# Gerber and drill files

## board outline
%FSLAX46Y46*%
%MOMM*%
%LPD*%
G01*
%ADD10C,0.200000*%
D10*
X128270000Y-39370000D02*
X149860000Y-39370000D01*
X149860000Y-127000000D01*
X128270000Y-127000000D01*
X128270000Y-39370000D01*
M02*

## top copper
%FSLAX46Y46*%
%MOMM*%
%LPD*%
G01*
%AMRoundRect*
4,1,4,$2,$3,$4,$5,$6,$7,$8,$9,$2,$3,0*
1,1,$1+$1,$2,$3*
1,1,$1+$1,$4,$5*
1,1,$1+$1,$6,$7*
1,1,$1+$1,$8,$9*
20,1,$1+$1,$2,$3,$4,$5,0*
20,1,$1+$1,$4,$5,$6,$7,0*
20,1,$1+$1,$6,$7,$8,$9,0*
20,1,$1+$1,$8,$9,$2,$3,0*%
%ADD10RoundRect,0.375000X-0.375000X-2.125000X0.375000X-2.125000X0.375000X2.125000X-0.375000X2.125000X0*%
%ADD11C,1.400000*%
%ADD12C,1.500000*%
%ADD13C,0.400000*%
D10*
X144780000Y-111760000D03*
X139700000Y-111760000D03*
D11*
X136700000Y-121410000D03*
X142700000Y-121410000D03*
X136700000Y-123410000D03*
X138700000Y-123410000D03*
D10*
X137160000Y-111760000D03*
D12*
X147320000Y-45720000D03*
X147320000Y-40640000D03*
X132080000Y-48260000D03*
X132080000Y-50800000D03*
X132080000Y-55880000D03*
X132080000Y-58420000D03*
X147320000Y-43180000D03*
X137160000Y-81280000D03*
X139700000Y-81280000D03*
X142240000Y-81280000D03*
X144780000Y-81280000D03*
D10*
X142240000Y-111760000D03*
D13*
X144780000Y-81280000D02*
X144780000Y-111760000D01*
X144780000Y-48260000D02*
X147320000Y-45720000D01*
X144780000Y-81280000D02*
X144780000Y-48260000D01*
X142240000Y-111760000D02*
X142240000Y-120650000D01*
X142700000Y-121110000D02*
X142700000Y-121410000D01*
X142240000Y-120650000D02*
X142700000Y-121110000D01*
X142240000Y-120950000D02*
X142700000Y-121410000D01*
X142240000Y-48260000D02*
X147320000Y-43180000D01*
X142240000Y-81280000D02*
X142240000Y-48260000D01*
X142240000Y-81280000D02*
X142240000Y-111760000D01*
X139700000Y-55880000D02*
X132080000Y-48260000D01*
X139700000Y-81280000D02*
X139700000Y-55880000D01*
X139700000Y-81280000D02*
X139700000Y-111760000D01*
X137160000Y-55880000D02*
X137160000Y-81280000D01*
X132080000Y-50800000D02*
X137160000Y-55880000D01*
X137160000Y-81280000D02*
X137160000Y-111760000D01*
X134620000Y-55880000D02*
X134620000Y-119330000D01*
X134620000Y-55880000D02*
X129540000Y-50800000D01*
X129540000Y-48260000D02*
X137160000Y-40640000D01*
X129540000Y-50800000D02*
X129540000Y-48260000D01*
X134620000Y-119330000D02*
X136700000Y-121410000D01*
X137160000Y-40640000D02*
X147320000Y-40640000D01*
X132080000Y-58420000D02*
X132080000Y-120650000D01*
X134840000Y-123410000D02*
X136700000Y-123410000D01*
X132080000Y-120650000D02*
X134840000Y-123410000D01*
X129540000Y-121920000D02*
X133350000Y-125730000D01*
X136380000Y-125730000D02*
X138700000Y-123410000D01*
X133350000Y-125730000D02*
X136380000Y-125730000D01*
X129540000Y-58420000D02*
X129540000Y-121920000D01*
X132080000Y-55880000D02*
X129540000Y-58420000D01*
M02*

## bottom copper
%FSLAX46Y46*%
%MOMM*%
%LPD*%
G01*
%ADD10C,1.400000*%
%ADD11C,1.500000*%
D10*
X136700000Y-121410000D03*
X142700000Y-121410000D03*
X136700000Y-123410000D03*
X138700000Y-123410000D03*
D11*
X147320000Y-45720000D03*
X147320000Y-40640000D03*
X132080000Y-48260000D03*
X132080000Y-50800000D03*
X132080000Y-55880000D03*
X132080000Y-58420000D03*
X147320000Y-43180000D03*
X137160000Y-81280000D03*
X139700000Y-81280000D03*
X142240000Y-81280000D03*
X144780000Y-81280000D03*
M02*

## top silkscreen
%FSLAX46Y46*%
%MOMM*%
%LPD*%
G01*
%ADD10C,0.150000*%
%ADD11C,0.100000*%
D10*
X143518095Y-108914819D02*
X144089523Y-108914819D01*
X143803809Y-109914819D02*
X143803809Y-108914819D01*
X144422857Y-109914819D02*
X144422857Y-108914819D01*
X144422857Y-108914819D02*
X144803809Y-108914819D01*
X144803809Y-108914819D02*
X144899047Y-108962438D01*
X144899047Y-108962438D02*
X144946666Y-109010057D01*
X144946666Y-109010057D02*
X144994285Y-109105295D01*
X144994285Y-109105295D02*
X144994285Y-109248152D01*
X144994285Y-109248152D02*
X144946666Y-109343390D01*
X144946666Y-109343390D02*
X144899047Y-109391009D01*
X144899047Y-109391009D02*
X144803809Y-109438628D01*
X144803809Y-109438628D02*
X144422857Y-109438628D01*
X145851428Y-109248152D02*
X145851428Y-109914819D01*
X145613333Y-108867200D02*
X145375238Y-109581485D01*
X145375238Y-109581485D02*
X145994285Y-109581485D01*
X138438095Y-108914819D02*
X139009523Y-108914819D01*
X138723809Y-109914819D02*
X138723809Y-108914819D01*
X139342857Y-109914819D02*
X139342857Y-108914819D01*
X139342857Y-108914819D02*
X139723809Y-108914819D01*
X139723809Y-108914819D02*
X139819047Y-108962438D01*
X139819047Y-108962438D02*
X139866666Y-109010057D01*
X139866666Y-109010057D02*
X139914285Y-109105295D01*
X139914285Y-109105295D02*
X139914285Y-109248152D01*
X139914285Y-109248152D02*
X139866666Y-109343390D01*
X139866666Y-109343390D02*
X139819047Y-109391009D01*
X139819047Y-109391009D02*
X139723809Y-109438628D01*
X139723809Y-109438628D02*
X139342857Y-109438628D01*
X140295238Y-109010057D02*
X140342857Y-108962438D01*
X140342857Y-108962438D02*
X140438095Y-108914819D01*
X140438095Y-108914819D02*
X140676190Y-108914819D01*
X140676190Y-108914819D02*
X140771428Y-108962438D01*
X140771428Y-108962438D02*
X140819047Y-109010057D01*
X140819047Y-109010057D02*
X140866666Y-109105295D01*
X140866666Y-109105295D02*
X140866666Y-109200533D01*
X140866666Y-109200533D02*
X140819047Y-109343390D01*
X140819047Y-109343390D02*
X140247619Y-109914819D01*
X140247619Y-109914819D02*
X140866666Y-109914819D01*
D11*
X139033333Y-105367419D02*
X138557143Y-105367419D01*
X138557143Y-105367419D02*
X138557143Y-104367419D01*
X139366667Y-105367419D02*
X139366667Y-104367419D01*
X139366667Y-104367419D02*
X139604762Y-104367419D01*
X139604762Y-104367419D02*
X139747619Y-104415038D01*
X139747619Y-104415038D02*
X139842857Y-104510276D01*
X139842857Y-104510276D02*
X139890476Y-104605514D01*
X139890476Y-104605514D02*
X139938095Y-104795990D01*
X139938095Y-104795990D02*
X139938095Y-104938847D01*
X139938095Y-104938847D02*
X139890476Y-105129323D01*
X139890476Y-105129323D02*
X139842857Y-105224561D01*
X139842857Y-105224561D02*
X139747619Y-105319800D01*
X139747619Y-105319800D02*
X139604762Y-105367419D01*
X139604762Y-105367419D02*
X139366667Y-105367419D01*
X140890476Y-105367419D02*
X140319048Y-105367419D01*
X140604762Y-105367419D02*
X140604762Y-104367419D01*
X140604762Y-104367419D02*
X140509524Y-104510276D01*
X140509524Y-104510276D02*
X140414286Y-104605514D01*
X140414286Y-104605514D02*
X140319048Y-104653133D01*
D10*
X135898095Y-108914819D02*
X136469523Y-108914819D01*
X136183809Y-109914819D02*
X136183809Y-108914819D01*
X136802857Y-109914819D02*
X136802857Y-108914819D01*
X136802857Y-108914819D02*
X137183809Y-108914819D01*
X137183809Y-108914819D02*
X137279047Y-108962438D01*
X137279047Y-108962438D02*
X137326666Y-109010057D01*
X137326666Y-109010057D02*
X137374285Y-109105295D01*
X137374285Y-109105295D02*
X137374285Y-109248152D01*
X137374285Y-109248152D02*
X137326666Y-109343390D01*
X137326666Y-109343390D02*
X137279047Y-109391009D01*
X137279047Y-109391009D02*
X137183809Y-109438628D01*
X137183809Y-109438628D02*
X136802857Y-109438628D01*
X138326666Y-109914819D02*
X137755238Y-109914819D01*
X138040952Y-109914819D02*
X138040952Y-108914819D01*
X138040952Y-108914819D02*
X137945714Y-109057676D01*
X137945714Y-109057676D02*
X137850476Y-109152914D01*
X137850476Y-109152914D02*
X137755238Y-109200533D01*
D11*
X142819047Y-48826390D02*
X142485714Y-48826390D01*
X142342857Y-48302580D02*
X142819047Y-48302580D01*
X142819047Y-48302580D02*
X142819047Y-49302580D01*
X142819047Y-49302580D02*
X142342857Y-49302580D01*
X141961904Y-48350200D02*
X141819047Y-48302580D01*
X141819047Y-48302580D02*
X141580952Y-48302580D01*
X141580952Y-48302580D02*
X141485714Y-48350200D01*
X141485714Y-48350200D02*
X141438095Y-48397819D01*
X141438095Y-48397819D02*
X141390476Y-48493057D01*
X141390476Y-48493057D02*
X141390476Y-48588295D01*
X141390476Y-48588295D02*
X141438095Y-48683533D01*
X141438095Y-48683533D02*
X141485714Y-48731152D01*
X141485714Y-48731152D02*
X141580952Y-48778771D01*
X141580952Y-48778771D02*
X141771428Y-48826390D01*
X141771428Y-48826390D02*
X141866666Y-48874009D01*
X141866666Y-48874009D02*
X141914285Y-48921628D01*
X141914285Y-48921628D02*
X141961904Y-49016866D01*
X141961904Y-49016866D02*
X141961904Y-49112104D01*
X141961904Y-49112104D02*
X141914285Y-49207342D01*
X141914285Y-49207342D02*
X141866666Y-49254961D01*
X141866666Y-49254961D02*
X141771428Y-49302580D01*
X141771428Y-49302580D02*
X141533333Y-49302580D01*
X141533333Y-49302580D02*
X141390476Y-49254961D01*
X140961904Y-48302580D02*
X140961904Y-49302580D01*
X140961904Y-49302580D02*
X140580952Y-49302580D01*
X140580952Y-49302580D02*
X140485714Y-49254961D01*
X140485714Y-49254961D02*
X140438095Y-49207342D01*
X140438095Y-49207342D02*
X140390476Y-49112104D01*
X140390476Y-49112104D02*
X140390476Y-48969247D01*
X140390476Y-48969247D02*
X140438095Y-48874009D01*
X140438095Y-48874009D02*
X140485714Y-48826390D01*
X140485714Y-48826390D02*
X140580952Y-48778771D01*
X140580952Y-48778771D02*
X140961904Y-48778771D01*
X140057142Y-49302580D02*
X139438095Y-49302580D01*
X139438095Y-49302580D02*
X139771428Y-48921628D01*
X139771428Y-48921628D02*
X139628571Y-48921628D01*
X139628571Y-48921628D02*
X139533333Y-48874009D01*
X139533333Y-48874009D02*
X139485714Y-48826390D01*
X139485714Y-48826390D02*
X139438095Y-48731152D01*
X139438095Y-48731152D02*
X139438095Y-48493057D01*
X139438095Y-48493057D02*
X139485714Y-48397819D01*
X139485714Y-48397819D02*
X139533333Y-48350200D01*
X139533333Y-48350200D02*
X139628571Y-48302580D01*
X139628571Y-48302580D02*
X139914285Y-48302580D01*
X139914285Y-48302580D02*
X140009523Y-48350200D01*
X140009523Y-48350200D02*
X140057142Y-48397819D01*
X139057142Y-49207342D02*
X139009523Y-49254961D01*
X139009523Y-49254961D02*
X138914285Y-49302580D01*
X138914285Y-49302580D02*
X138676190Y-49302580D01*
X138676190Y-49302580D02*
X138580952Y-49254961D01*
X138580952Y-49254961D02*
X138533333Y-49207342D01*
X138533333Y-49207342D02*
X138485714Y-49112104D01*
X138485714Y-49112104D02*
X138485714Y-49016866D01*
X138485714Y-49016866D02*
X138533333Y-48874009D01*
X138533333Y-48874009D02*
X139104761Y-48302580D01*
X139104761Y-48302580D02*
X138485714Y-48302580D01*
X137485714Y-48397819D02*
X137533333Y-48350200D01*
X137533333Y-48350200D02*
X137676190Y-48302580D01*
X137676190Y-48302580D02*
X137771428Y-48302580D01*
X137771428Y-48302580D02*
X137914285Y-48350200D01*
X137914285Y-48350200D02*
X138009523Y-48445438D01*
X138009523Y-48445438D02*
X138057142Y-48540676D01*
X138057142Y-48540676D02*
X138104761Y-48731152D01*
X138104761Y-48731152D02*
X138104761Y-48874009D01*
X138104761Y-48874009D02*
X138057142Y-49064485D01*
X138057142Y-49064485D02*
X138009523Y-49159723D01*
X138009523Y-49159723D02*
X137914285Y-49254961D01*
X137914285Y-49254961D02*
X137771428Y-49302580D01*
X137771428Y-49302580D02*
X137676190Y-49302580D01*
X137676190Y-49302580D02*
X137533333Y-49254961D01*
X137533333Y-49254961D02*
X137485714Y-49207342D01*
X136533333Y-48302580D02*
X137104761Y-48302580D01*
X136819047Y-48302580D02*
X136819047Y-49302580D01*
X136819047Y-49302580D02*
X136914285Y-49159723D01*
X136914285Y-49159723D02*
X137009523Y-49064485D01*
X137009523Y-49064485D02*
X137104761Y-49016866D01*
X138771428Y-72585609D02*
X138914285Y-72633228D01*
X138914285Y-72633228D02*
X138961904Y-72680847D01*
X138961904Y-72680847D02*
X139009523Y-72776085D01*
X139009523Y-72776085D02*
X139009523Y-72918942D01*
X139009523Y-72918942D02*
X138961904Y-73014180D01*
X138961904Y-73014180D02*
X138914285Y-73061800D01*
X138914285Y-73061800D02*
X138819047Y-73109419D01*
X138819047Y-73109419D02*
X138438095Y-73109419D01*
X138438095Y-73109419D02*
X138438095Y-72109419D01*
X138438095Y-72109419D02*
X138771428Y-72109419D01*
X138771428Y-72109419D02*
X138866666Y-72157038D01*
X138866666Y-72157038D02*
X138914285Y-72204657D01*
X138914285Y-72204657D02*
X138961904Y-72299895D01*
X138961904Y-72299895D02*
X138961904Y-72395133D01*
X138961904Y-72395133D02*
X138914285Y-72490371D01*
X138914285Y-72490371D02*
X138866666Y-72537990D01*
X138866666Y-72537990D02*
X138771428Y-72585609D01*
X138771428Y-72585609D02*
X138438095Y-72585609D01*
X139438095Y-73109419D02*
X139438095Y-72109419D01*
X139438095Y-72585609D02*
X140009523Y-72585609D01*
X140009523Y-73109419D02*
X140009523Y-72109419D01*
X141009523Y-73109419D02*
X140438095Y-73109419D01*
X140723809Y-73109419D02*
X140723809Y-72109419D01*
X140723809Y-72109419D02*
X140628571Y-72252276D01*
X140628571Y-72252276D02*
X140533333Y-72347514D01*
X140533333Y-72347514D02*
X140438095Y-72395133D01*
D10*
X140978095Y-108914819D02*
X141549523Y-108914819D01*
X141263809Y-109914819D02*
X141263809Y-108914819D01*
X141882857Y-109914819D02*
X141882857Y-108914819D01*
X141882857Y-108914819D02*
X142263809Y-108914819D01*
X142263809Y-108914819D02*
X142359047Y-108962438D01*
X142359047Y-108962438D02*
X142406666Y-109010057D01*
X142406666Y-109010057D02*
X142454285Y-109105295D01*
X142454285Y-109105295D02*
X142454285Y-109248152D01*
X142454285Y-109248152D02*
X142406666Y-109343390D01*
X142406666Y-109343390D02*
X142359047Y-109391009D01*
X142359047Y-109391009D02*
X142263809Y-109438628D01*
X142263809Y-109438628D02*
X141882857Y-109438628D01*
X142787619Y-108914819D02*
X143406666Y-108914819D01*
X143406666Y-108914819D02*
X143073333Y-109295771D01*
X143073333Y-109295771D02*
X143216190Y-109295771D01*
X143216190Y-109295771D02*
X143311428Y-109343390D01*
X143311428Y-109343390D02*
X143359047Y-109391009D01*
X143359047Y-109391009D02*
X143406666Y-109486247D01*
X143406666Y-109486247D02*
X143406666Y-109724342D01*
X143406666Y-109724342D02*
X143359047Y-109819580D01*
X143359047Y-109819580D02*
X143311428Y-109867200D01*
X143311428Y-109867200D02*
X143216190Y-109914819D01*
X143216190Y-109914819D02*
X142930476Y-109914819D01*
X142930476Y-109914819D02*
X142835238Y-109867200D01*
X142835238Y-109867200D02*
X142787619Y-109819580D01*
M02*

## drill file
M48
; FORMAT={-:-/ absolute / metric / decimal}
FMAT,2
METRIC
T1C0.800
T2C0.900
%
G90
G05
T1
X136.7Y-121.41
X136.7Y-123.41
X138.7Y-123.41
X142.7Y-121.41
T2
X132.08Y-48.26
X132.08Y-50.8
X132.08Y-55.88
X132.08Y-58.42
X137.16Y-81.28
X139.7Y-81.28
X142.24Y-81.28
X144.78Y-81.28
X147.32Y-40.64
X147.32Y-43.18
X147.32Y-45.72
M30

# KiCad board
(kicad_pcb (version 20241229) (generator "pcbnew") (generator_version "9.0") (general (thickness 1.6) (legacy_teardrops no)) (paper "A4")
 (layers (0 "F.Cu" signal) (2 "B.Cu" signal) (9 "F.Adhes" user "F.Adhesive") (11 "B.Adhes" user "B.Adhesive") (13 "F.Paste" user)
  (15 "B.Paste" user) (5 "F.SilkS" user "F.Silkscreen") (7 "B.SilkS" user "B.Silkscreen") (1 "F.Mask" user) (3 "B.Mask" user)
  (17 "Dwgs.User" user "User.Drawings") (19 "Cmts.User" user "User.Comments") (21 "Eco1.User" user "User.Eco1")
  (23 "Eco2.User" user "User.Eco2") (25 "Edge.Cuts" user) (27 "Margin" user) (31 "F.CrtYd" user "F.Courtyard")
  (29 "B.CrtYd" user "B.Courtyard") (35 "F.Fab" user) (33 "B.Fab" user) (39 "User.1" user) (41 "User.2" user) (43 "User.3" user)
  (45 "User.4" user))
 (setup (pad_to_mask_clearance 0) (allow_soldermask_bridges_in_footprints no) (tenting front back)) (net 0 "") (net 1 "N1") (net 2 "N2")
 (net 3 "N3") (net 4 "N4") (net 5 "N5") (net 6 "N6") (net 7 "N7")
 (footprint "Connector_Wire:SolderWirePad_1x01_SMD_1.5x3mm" (layer "F.Cu") (at 144.78 111.76)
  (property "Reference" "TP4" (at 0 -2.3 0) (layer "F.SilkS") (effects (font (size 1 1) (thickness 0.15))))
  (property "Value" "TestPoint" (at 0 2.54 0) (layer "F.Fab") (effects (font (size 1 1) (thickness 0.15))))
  (pad "1" smd roundrect (at 0 0) (size 1.5 5) (layers "F.Cu" "F.Mask") (roundrect_rratio 0.25) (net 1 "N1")))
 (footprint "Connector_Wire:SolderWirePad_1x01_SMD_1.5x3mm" (layer "F.Cu") (at 139.7 111.76)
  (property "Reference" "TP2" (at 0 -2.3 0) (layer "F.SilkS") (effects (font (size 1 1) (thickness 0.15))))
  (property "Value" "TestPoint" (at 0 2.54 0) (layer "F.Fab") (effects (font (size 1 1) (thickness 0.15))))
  (pad "1" smd roundrect (at 0 0) (size 1.5 5) (layers "F.Cu" "F.Mask") (roundrect_rratio 0.25) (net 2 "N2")))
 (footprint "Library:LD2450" (layer "F.Cu") (at 139.7 105.41)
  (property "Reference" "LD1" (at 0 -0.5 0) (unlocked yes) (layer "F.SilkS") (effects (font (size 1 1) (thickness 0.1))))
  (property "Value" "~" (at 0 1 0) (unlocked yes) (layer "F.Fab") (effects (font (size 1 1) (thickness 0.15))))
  (pad "1" thru_hole circle (at -3 16 90) (size 1.4 1.4) (drill 0.8) (layers "*.Cu" "*.Mask") (remove_unused_layers yes)
   (keep_end_layers yes) (zone_layer_connections) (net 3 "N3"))
  (pad "2" thru_hole circle (at 3 16 90) (size 1.4 1.4) (drill 0.8) (layers "*.Cu" "*.Mask") (remove_unused_layers yes)
   (keep_end_layers yes) (zone_layer_connections) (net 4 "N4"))
  (pad "3" thru_hole circle (at -3 18 90) (size 1.4 1.4) (drill 0.8) (layers "*.Cu" "*.Mask") (remove_unused_layers yes)
   (keep_end_layers yes) (zone_layer_connections) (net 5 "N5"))
  (pad "4" thru_hole circle (at -1 18 90) (size 1.4 1.4) (drill 0.8) (layers "*.Cu" "*.Mask") (remove_unused_layers yes)
   (keep_end_layers yes) (zone_layer_connections) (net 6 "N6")))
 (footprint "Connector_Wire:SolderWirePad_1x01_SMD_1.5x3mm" (layer "F.Cu") (at 137.16 111.76)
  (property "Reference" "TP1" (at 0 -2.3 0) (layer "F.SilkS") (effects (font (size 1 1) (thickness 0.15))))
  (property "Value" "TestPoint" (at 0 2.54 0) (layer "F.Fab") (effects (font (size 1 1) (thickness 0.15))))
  (pad "1" smd roundrect (at 0 0) (size 1.5 5) (layers "F.Cu" "F.Mask") (roundrect_rratio 0.25) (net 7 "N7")))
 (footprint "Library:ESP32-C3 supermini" (layer "F.Cu") (at 139.7 50.8 180)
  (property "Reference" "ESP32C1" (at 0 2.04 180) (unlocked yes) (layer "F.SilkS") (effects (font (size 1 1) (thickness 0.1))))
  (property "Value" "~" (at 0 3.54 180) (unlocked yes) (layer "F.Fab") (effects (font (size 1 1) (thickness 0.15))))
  (pad "3.3V" thru_hole circle (at -7.62 5.08 180) (size 1.5 1.5) (drill 0.9) (layers "*.Cu" "*.Mask") (remove_unused_layers yes)
   (keep_end_layers yes) (zone_layer_connections) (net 1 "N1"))
  (pad "5V" thru_hole circle (at -7.62 10.16 180) (size 1.5 1.5) (drill 0.9) (layers "*.Cu" "*.Mask") (remove_unused_layers yes)
   (keep_end_layers yes) (zone_layer_connections) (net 3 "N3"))
  (pad "8" thru_hole circle (at 7.62 2.54 180) (size 1.5 1.5) (drill 0.9) (layers "*.Cu" "*.Mask") (remove_unused_layers yes)
   (keep_end_layers yes) (zone_layer_connections) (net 2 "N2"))
  (pad "9" thru_hole circle (at 7.62 0 180) (size 1.5 1.5) (drill 0.9) (layers "*.Cu" "*.Mask") (remove_unused_layers yes)
   (keep_end_layers yes) (zone_layer_connections) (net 7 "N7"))
  (pad "20" thru_hole circle (at 7.62 -5.08 180) (size 1.5 1.5) (drill 0.9) (layers "*.Cu" "*.Mask") (remove_unused_layers yes)
   (keep_end_layers yes) (zone_layer_connections) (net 6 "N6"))
  (pad "21" thru_hole circle (at 7.62 -7.62 180) (size 1.5 1.5) (drill 0.9) (layers "*.Cu" "*.Mask") (remove_unused_layers yes)
   (keep_end_layers yes) (zone_layer_connections) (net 5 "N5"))
  (pad "GND" thru_hole circle (at -7.62 7.62 180) (size 1.5 1.5) (drill 0.9) (layers "*.Cu" "*.Mask") (remove_unused_layers yes)
   (keep_end_layers yes) (zone_layer_connections) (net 4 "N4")))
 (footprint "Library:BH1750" (layer "F.Cu") (at 139.7 73.152)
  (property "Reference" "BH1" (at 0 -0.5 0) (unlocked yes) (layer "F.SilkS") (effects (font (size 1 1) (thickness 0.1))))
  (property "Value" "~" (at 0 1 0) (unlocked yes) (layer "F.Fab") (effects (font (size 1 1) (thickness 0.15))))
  (pad "1" thru_hole circle (at -2.54 8.128 90) (size 1.5 1.5) (drill 0.9) (layers "*.Cu" "*.Mask") (remove_unused_layers yes)
   (keep_end_layers yes) (zone_layer_connections) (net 7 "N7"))
  (pad "2" thru_hole circle (at 0 8.128 90) (size 1.5 1.5) (drill 0.9) (layers "*.Cu" "*.Mask") (remove_unused_layers yes)
   (keep_end_layers yes) (zone_layer_connections) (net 2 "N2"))
  (pad "3" thru_hole circle (at 2.54 8.128 90) (size 1.5 1.5) (drill 0.9) (layers "*.Cu" "*.Mask") (remove_unused_layers yes)
   (keep_end_layers yes) (zone_layer_connections) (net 4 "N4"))
  (pad "4" thru_hole circle (at 5.08 8.128 90) (size 1.5 1.5) (drill 0.9) (layers "*.Cu" "*.Mask") (remove_unused_layers yes)
   (keep_end_layers yes) (zone_layer_connections) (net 1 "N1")))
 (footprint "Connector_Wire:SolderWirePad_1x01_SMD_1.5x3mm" (layer "F.Cu") (at 142.24 111.76)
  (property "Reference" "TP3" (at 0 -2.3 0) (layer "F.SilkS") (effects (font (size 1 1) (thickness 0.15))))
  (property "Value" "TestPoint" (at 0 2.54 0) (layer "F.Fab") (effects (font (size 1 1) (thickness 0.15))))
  (pad "1" smd roundrect (at 0 0) (size 1.5 5) (layers "F.Cu" "F.Mask") (roundrect_rratio 0.25) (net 4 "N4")))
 (gr_rect (start 128.27 39.37) (end 149.86 127) (stroke (width 0.2) (type solid)) (fill no) (layer "Edge.Cuts"))
 (segment (start 144.78 81.28) (end 144.78 111.76) (width 0.4) (layer "F.Cu") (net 1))
 (segment (start 144.78 48.26) (end 147.32 45.72) (width 0.4) (layer "F.Cu") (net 1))
 (segment (start 144.78 81.28) (end 144.78 48.26) (width 0.4) (layer "F.Cu") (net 1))
 (segment (start 142.24 111.76) (end 142.24 120.65) (width 0.4) (layer "F.Cu") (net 4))
 (segment (start 142.7 121.11) (end 142.7 121.41) (width 0.4) (layer "F.Cu") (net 4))
 (segment (start 142.24 120.65) (end 142.7 121.11) (width 0.4) (layer "F.Cu") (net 4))
 (segment (start 142.24 120.95) (end 142.7 121.41) (width 0.4) (layer "F.Cu") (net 4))
 (segment (start 142.24 48.26) (end 147.32 43.18) (width 0.4) (layer "F.Cu") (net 4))
 (segment (start 142.24 81.28) (end 142.24 48.26) (width 0.4) (layer "F.Cu") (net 4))
 (segment (start 142.24 81.28) (end 142.24 111.76) (width 0.4) (layer "F.Cu") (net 4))
 (segment (start 139.7 55.88) (end 132.08 48.26) (width 0.4) (layer "F.Cu") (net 2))
 (segment (start 139.7 81.28) (end 139.7 55.88) (width 0.4) (layer "F.Cu") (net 2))
 (segment (start 139.7 81.28) (end 139.7 111.76) (width 0.4) (layer "F.Cu") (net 2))
 (segment (start 137.16 55.88) (end 137.16 81.28) (width 0.4) (layer "F.Cu") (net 7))
 (segment (start 132.08 50.8) (end 137.16 55.88) (width 0.4) (layer "F.Cu") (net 7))
 (segment (start 137.16 81.28) (end 137.16 111.76) (width 0.4) (layer "F.Cu") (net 7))
 (segment (start 134.62 55.88) (end 134.62 119.33) (width 0.4) (layer "F.Cu") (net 3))
 (segment (start 134.62 55.88) (end 129.54 50.8) (width 0.4) (layer "F.Cu") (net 3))
 (segment (start 129.54 48.26) (end 137.16 40.64) (width 0.4) (layer "F.Cu") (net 3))
 (segment (start 129.54 50.8) (end 129.54 48.26) (width 0.4) (layer "F.Cu") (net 3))
 (segment (start 134.62 119.33) (end 136.7 121.41) (width 0.4) (layer "F.Cu") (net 3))
 (segment (start 137.16 40.64) (end 147.32 40.64) (width 0.4) (layer "F.Cu") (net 3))
 (segment (start 132.08 58.42) (end 132.08 120.65) (width 0.4) (layer "F.Cu") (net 5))
 (segment (start 134.84 123.41) (end 136.7 123.41) (width 0.4) (layer "F.Cu") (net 5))
 (segment (start 132.08 120.65) (end 134.84 123.41) (width 0.4) (layer "F.Cu") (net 5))
 (segment (start 129.54 121.92) (end 133.35 125.73) (width 0.4) (layer "F.Cu") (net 6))
 (segment (start 136.38 125.73) (end 138.7 123.41) (width 0.4) (layer "F.Cu") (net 6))
 (segment (start 133.35 125.73) (end 136.38 125.73) (width 0.4) (layer "F.Cu") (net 6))
 (segment (start 129.54 58.42) (end 129.54 121.92) (width 0.4) (layer "F.Cu") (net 6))
 (segment (start 132.08 55.88) (end 129.54 58.42) (width 0.4) (layer "F.Cu") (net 6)))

